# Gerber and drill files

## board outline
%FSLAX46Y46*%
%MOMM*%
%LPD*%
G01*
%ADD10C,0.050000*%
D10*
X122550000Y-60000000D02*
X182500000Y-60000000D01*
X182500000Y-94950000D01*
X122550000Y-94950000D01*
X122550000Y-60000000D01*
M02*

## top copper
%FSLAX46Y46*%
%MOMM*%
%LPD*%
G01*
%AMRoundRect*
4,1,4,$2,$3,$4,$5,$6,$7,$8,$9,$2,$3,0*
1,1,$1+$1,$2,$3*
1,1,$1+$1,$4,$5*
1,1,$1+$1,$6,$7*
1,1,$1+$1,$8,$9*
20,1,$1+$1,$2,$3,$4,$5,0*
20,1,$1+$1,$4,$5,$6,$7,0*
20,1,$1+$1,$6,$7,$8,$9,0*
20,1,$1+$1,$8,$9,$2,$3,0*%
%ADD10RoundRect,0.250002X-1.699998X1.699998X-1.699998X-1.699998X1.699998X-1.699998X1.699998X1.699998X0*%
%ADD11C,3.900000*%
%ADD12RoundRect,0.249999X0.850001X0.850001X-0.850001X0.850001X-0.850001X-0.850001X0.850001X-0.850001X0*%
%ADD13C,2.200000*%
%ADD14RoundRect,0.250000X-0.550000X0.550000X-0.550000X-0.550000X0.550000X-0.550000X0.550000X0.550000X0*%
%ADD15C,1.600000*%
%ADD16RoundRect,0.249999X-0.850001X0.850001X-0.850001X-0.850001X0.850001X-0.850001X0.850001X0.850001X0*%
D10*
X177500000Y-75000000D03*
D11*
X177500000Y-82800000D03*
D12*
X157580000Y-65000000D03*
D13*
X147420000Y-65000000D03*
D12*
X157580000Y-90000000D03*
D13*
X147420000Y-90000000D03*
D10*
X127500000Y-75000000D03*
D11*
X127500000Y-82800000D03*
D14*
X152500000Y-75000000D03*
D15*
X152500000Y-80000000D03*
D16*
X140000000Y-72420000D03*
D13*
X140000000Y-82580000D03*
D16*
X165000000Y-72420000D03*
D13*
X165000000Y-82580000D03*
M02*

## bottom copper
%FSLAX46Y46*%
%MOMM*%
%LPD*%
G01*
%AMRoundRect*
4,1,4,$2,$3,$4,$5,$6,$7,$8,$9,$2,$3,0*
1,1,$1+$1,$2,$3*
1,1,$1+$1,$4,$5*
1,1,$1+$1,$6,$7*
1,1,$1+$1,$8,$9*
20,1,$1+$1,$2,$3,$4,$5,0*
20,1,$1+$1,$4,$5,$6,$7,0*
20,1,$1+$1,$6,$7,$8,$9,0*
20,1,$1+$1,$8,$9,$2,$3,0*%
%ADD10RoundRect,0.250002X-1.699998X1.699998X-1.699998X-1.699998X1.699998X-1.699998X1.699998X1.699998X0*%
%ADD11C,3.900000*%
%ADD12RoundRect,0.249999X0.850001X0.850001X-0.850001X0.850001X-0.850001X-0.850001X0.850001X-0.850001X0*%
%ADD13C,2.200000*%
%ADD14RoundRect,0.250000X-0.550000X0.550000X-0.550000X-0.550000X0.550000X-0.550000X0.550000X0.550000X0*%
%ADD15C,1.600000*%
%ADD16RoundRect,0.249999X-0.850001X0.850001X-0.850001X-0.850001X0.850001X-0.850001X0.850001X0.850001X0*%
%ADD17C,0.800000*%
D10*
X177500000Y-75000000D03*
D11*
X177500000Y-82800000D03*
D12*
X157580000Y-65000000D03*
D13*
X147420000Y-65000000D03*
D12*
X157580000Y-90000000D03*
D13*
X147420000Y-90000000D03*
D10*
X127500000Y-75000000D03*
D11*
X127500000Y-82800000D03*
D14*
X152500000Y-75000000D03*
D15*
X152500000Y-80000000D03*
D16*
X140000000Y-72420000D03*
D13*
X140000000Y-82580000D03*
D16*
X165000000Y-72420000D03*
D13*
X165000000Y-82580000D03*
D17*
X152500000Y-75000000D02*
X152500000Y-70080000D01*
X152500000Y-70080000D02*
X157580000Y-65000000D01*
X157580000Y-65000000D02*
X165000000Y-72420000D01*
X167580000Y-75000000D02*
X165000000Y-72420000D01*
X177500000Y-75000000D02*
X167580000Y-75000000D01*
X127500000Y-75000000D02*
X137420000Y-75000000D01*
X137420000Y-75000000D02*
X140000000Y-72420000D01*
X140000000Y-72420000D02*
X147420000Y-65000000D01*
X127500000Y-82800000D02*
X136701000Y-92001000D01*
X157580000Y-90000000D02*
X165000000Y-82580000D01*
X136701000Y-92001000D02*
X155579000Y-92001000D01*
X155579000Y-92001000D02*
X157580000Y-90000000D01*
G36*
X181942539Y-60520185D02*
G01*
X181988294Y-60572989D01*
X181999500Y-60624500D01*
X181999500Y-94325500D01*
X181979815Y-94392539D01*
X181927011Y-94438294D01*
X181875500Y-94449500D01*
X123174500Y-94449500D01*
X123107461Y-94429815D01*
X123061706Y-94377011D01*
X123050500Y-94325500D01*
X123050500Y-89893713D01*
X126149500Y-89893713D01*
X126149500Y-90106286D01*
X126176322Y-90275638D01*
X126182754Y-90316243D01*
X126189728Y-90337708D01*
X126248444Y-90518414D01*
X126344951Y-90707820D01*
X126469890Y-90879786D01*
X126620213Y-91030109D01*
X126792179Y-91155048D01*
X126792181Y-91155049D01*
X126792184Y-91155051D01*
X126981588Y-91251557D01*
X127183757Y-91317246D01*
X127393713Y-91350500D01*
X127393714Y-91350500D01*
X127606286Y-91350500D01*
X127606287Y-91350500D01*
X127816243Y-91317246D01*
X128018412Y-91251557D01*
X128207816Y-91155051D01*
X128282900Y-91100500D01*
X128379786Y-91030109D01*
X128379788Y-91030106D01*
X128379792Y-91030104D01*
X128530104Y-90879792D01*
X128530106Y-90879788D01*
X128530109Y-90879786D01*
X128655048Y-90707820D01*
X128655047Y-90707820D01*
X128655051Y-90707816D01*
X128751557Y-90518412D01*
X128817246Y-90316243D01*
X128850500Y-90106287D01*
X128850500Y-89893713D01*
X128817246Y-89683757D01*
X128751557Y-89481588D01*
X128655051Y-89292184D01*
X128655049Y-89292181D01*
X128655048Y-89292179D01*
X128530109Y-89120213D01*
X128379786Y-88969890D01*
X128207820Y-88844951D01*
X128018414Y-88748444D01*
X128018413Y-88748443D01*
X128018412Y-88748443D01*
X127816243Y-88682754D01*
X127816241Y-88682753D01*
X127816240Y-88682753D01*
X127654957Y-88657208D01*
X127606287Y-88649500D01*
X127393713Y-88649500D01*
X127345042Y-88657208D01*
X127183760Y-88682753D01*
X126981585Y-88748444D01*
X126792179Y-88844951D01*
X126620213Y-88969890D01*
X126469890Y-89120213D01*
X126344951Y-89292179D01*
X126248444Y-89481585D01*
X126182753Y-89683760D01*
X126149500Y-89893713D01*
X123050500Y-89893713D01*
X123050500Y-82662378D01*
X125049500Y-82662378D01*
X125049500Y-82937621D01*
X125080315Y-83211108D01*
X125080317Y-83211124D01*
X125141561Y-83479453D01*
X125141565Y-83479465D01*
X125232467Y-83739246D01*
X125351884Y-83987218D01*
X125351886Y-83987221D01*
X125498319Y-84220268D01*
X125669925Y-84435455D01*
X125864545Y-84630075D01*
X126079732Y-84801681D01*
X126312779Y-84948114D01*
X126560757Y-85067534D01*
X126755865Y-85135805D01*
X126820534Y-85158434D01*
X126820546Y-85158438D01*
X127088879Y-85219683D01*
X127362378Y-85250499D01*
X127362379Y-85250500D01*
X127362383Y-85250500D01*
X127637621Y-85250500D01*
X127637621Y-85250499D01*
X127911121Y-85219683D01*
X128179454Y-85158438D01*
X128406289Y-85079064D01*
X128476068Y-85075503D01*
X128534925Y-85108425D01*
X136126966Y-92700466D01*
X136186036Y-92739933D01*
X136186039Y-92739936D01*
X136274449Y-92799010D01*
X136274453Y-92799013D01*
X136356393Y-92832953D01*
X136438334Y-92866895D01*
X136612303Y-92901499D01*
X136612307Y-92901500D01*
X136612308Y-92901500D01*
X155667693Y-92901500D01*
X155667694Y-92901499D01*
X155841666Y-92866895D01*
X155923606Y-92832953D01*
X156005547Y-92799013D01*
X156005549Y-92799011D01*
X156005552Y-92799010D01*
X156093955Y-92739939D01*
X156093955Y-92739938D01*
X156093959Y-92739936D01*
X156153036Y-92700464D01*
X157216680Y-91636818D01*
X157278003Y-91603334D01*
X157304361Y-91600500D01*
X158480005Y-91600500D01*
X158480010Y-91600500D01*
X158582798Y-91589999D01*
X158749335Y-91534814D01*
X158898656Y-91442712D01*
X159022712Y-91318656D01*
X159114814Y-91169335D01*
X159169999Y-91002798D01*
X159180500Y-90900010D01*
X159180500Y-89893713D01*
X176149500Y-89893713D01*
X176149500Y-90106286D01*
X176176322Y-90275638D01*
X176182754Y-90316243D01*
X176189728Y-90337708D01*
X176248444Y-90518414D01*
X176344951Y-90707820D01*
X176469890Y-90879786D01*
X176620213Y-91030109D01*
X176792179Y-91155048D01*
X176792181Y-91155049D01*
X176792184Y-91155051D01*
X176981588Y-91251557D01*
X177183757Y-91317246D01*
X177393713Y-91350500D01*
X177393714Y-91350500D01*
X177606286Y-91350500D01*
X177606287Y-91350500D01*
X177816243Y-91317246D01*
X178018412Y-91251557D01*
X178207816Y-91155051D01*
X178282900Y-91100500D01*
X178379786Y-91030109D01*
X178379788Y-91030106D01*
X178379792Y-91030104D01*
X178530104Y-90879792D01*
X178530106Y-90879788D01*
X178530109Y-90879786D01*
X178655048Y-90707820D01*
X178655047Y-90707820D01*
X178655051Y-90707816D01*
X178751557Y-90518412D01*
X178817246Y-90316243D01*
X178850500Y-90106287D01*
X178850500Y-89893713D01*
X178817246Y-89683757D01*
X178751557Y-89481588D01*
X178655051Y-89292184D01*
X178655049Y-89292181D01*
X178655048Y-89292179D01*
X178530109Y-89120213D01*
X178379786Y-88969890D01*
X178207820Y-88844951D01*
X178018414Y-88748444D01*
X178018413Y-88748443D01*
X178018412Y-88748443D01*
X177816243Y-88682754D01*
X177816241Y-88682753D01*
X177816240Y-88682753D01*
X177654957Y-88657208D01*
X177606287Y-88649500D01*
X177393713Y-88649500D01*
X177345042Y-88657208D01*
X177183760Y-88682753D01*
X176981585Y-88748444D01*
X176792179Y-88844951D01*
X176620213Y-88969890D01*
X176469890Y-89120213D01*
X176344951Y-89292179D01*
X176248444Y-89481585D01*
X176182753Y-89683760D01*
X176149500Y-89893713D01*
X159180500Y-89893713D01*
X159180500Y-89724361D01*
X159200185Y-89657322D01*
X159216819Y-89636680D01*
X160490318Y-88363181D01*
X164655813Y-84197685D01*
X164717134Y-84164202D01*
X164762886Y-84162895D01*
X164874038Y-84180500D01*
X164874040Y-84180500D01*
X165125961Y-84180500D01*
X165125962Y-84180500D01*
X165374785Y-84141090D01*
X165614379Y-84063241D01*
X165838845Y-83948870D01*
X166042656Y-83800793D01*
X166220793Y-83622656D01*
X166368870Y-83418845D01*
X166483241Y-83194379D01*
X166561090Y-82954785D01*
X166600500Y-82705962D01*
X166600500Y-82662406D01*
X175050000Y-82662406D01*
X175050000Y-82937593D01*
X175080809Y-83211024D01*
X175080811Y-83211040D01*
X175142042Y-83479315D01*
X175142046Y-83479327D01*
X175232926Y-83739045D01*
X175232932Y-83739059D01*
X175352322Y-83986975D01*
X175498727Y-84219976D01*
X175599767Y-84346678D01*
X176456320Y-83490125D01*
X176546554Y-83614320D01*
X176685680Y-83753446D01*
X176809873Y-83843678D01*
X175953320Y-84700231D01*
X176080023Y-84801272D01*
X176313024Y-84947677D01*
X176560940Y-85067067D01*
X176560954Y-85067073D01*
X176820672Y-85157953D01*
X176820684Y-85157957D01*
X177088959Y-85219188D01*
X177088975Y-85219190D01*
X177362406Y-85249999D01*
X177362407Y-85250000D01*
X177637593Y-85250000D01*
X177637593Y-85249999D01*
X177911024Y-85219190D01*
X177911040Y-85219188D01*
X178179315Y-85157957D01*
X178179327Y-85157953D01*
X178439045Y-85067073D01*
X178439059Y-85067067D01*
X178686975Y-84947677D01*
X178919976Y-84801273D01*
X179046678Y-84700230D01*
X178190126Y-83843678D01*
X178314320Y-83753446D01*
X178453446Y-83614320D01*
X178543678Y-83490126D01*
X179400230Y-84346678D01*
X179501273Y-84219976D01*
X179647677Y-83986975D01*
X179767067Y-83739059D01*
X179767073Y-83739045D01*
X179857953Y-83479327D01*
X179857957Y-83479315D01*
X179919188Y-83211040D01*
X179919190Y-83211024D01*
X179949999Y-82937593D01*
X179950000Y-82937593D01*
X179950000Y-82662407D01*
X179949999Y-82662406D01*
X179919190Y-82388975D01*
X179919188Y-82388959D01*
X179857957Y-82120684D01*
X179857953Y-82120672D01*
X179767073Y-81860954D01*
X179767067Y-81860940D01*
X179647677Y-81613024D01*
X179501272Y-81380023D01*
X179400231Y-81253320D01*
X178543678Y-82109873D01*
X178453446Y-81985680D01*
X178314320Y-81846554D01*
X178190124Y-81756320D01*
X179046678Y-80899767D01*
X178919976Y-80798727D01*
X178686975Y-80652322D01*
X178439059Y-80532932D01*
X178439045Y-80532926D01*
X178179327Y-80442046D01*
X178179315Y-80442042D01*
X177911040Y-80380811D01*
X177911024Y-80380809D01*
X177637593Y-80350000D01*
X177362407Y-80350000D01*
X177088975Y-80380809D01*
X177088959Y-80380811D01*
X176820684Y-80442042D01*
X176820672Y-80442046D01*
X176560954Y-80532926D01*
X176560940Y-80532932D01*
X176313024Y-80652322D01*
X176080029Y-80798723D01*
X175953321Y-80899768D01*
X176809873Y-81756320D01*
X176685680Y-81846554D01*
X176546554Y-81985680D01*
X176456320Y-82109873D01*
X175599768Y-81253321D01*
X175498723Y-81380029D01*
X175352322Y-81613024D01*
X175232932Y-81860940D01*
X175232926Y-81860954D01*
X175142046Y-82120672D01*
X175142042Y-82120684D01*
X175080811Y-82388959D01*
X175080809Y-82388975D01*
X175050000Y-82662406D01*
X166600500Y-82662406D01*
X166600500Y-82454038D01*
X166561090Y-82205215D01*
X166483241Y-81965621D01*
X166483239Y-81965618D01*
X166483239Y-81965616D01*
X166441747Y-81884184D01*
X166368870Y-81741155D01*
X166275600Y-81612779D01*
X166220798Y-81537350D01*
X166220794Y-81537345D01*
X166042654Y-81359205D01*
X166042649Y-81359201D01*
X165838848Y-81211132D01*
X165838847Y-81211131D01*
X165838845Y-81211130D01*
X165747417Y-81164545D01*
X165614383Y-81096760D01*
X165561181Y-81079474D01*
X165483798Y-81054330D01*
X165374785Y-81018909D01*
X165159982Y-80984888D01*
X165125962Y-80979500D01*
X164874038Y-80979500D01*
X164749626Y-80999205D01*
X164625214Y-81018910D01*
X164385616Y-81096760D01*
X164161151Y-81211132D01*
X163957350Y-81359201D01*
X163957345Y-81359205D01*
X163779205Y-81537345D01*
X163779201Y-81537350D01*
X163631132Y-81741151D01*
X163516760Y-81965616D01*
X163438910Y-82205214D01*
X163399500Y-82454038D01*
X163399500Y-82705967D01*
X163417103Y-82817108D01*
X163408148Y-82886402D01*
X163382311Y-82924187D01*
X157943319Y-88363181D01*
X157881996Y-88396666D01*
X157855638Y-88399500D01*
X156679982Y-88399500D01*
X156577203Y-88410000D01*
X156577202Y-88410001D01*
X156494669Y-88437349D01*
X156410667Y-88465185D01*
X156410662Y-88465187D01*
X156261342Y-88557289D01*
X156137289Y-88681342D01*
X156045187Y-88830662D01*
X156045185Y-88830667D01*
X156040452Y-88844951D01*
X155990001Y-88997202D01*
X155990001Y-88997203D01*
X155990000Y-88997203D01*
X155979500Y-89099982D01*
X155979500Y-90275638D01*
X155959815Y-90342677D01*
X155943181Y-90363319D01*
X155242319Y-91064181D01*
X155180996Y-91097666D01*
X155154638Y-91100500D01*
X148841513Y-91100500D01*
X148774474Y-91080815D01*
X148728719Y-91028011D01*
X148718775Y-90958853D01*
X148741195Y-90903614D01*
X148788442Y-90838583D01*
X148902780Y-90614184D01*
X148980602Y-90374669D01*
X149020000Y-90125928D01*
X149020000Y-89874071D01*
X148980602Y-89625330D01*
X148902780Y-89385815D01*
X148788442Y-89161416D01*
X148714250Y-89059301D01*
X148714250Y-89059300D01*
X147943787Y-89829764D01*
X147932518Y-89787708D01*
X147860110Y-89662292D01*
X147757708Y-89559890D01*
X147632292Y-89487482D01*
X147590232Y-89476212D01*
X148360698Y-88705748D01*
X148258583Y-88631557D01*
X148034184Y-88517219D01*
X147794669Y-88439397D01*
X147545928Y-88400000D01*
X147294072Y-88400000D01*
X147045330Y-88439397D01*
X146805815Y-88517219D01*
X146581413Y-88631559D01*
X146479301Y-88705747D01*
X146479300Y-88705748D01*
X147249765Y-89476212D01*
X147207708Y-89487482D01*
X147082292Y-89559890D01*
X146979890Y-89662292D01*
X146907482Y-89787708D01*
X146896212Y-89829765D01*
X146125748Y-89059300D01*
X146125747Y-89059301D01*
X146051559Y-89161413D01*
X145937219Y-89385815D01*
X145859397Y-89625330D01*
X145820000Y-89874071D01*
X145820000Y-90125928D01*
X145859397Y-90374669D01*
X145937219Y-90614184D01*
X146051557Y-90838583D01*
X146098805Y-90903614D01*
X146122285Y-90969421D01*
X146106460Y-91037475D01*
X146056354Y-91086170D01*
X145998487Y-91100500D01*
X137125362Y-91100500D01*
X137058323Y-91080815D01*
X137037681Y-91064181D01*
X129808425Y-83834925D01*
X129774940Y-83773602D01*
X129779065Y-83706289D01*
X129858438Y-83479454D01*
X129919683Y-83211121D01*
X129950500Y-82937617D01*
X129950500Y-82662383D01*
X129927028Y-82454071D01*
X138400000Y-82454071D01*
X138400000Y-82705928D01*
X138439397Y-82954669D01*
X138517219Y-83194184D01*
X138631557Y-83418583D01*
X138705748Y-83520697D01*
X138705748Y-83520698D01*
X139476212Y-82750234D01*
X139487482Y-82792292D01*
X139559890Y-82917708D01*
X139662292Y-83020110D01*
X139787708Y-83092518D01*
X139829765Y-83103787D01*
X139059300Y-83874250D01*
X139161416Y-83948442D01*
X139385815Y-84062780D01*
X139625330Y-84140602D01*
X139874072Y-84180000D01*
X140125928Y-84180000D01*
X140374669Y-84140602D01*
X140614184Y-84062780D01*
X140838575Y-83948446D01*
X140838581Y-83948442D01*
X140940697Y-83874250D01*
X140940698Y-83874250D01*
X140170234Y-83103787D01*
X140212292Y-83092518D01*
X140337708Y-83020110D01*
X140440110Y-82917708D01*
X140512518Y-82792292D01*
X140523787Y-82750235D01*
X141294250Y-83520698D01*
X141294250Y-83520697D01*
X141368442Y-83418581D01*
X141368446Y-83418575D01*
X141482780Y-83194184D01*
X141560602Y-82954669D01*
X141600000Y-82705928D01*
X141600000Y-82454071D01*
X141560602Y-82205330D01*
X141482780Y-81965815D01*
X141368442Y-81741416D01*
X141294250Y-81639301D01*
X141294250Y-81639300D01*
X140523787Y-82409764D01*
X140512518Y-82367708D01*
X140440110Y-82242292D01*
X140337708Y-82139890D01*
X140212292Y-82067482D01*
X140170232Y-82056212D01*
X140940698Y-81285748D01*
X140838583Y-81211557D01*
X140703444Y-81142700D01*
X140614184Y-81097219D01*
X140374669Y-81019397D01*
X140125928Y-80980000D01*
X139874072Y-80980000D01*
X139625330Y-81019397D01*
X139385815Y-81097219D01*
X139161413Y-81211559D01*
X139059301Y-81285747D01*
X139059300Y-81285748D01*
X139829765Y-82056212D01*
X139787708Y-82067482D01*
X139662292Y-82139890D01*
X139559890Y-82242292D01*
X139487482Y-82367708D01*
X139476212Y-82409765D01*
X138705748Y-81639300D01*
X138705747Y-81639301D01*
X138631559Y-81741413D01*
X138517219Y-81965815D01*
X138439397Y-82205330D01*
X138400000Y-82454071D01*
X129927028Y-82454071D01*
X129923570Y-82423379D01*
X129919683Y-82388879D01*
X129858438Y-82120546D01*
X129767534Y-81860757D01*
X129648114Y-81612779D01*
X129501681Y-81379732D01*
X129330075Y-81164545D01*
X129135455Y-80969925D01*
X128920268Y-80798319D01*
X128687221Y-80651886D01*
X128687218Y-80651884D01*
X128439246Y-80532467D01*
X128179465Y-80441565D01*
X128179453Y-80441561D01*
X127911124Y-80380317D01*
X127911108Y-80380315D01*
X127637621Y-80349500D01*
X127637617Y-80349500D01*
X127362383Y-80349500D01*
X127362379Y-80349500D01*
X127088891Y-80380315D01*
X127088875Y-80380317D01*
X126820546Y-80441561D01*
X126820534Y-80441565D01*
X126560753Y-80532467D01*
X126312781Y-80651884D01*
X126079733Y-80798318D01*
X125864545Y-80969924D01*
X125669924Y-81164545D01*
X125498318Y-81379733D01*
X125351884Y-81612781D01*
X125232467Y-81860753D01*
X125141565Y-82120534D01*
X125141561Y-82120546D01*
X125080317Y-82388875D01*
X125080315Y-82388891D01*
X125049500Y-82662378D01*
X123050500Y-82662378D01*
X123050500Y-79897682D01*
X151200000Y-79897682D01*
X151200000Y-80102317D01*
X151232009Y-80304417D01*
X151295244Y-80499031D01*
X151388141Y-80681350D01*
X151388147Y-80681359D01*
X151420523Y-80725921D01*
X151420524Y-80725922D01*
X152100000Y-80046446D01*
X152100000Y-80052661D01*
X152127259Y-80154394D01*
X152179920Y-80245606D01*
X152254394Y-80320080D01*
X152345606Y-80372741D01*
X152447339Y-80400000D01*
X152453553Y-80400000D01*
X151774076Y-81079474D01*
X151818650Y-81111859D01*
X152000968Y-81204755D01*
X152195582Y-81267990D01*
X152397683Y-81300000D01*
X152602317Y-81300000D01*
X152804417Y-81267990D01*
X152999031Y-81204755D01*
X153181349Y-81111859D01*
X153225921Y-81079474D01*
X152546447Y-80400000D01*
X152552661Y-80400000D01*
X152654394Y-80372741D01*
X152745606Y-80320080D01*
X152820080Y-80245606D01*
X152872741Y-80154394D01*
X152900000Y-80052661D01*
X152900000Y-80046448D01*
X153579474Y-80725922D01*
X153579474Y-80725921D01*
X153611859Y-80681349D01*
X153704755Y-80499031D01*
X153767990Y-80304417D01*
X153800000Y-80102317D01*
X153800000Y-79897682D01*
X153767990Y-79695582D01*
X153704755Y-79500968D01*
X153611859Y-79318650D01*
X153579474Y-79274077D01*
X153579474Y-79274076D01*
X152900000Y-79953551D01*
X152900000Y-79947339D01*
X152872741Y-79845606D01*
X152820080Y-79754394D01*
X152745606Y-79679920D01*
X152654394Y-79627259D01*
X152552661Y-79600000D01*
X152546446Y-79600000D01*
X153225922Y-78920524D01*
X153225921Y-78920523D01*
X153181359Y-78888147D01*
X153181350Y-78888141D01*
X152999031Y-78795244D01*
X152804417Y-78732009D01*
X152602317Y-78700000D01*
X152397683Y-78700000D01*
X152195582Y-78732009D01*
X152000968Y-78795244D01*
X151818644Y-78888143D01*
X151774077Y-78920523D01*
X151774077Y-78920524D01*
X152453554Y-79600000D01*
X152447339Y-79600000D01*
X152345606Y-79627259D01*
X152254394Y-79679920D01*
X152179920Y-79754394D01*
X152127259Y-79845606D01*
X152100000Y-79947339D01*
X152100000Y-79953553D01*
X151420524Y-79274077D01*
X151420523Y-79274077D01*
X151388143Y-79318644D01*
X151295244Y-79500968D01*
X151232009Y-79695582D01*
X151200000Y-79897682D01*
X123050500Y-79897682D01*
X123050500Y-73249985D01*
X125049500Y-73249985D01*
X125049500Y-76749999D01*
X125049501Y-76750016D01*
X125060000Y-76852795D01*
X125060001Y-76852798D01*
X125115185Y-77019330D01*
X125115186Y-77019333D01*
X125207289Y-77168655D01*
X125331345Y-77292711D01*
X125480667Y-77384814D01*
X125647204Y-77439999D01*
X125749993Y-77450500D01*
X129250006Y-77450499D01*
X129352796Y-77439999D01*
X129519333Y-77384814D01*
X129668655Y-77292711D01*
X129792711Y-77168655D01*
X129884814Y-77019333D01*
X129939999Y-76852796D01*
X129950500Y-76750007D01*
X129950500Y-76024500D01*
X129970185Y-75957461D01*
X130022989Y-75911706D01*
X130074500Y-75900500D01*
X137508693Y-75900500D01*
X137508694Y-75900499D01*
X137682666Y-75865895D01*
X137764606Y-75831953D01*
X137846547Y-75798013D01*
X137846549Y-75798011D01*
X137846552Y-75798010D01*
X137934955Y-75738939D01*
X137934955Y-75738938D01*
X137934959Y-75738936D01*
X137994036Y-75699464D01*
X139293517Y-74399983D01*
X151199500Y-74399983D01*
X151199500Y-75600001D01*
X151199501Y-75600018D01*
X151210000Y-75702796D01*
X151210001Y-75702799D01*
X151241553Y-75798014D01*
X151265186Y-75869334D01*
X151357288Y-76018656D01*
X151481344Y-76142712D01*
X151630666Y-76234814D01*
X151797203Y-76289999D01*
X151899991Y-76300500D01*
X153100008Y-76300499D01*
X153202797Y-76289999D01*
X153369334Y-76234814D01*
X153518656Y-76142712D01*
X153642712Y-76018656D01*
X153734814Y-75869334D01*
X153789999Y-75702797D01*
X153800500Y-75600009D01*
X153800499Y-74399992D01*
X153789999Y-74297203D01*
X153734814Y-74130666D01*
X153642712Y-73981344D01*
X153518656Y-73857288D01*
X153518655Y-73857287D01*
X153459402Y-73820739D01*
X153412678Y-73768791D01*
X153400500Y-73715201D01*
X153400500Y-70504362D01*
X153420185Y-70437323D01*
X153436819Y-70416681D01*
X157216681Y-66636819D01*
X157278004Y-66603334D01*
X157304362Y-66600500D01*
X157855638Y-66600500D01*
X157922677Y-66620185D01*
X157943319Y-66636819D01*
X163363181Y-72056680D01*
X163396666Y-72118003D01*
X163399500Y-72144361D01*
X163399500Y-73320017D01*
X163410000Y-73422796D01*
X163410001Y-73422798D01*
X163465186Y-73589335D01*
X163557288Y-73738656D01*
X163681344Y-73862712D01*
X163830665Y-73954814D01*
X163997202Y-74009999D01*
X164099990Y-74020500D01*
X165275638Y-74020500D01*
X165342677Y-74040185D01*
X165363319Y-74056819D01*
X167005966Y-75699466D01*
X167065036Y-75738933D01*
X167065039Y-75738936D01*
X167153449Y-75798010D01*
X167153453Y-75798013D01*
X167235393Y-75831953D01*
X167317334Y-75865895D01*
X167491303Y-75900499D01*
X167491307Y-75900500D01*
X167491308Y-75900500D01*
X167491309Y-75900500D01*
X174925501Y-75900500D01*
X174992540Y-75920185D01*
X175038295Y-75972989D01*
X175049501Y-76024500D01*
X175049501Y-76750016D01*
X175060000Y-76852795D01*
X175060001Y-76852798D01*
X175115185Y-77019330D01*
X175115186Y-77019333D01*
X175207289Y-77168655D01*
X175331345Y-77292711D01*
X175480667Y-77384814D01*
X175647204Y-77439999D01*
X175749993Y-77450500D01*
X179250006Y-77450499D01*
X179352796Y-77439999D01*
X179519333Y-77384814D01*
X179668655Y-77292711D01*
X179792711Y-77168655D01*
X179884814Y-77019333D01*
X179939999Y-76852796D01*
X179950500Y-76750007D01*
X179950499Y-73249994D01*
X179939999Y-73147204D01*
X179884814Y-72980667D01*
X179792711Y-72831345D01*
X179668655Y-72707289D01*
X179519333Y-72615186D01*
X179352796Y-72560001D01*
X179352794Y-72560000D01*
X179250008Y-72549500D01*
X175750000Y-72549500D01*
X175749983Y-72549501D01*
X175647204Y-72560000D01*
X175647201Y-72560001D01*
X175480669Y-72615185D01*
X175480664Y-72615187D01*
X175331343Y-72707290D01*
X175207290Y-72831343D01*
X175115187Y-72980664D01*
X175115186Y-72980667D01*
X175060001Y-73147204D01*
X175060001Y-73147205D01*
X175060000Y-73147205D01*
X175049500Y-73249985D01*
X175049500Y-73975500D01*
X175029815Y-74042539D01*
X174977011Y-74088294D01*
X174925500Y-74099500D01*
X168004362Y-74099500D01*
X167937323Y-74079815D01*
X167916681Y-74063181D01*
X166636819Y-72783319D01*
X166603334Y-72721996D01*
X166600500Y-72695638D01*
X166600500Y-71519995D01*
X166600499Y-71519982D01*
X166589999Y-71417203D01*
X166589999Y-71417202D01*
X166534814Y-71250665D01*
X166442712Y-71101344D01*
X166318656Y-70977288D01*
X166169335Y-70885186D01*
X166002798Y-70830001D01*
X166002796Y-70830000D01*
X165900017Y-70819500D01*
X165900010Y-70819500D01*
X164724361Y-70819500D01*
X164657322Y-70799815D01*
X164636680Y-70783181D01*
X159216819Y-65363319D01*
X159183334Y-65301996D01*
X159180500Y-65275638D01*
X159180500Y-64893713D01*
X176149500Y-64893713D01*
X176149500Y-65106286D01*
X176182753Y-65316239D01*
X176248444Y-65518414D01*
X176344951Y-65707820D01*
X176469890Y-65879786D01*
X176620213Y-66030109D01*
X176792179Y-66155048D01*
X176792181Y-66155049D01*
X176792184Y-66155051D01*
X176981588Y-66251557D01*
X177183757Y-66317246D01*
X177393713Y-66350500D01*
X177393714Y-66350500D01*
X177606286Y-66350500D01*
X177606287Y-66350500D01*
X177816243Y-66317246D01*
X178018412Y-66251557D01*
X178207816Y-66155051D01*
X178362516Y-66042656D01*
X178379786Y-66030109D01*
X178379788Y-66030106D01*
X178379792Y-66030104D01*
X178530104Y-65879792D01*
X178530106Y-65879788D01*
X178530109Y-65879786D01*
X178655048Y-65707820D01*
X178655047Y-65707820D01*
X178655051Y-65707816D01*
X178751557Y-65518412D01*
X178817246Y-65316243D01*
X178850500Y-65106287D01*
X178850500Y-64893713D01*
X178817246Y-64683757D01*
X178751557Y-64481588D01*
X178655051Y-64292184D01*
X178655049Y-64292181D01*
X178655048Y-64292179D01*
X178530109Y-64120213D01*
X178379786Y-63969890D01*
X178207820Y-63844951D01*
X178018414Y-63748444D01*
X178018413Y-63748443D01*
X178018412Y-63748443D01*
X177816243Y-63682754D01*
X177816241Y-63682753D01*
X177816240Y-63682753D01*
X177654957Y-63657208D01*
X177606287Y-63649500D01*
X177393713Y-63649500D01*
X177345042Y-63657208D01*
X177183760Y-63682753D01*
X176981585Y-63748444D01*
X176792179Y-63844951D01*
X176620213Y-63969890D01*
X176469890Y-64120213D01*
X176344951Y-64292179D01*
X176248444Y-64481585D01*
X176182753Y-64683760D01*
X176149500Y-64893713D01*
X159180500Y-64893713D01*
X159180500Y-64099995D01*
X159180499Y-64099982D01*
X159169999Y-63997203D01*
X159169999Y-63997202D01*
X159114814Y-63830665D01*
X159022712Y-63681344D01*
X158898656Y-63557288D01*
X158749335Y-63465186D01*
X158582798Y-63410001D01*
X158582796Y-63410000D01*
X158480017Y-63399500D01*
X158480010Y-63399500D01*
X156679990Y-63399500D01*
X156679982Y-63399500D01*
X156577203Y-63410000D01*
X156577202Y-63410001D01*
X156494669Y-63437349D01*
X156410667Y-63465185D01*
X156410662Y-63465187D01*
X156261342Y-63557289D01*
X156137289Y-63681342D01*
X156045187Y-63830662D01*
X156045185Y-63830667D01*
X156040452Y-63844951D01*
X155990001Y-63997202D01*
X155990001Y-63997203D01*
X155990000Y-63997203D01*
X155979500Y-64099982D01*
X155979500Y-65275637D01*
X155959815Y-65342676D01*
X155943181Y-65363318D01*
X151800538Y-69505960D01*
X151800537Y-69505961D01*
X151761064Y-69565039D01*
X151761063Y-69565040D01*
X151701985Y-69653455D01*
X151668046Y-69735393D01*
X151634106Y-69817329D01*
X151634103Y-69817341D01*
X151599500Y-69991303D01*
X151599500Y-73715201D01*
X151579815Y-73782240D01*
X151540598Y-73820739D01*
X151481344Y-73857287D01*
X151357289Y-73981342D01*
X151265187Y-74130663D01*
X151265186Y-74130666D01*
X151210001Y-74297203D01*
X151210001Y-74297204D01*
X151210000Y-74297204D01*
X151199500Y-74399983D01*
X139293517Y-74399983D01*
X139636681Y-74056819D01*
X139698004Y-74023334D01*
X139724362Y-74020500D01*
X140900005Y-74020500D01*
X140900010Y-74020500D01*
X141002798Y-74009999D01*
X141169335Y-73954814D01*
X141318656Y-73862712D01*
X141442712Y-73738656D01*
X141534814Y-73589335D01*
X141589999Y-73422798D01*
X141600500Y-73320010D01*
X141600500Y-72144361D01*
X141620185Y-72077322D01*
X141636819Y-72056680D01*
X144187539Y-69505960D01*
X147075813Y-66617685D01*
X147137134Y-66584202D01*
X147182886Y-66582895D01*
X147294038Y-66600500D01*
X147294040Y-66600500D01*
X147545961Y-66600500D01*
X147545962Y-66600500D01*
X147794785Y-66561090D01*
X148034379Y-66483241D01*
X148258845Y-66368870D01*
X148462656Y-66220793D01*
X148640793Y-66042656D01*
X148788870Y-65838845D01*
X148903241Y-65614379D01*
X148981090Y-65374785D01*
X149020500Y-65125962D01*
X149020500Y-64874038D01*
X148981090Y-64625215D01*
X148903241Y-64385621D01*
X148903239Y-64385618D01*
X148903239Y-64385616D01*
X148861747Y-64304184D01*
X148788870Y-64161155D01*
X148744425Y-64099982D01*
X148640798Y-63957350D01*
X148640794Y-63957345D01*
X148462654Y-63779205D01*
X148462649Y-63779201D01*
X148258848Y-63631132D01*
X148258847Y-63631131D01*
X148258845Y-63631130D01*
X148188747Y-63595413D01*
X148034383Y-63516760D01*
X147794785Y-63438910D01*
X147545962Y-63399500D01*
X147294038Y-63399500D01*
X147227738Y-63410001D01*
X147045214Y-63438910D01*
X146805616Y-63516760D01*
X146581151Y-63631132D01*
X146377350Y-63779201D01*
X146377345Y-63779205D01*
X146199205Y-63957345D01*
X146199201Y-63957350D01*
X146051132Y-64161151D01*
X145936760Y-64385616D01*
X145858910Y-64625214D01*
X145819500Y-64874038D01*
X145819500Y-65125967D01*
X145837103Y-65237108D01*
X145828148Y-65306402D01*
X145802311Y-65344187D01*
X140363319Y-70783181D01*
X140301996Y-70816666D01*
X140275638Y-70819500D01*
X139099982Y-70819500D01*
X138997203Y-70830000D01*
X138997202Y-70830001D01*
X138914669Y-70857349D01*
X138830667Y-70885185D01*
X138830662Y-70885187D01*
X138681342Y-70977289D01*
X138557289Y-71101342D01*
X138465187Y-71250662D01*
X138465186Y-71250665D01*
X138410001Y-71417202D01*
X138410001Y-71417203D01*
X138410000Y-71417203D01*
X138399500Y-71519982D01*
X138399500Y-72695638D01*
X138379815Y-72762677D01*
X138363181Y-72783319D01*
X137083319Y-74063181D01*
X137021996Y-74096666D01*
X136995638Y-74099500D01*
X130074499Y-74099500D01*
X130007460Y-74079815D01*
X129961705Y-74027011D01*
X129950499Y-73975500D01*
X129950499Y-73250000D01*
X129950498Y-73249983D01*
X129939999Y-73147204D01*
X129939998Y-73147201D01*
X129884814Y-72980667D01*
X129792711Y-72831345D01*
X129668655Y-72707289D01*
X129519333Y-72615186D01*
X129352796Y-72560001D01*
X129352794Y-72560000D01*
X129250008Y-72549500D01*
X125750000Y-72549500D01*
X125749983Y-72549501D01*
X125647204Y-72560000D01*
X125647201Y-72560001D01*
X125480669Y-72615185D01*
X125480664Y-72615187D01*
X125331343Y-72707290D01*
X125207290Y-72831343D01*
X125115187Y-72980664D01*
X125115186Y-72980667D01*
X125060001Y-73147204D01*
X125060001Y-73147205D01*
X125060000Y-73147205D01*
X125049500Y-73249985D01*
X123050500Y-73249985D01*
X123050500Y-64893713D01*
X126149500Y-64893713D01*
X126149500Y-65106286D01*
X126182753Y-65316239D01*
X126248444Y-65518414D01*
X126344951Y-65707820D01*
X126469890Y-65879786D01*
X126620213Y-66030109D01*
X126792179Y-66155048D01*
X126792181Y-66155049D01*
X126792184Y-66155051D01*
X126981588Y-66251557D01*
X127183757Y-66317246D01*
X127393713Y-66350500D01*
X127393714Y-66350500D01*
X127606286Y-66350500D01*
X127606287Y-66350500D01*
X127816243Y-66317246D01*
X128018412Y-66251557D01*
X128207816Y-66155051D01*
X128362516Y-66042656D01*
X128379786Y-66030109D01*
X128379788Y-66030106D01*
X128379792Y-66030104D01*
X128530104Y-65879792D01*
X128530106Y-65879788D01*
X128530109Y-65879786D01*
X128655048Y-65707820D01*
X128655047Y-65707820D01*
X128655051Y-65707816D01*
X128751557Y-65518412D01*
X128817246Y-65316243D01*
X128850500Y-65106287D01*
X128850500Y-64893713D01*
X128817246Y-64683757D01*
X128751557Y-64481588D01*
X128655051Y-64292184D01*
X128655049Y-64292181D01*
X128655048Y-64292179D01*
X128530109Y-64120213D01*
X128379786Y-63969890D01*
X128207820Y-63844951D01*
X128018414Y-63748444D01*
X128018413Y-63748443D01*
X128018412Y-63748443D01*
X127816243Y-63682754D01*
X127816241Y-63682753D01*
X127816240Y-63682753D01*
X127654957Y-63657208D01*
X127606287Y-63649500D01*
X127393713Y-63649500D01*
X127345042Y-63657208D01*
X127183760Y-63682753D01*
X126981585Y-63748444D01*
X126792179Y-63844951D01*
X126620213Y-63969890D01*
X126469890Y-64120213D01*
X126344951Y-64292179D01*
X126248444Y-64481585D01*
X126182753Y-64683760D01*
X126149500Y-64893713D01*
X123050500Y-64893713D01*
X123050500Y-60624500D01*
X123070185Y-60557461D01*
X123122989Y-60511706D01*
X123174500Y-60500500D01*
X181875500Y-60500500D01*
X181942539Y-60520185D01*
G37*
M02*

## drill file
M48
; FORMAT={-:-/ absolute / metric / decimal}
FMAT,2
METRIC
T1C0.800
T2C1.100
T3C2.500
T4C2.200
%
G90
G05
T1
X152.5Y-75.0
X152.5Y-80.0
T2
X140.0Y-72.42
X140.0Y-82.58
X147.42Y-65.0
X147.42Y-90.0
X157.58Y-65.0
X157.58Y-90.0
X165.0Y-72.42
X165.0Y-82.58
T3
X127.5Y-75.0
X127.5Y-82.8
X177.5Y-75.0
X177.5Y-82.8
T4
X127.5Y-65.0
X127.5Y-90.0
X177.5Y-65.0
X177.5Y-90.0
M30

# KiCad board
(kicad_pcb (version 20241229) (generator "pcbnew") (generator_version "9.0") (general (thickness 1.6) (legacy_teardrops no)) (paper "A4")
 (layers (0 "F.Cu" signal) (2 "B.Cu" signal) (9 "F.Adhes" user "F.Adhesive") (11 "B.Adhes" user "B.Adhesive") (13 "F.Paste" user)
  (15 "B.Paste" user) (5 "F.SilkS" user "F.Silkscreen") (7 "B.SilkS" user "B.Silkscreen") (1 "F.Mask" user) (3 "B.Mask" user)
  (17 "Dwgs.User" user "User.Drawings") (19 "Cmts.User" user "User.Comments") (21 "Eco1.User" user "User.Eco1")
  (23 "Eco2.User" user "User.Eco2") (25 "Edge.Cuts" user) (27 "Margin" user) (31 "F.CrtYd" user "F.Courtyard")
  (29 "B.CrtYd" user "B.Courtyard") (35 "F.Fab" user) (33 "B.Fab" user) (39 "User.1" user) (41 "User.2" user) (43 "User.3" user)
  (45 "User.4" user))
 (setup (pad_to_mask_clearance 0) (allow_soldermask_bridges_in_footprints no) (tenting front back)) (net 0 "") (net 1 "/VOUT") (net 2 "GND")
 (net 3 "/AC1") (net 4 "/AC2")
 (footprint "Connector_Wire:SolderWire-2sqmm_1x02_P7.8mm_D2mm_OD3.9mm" (layer "F.Cu") (at 177.5 75 -90)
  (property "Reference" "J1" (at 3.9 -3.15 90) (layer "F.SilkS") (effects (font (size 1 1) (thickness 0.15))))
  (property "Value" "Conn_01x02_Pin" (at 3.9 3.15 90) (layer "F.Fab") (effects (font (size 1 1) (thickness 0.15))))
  (pad "1" thru_hole roundrect (at 0 0 270) (size 3.9 3.9) (drill 2.5) (layers "*.Cu" "*.Mask") (remove_unused_layers no)
   (roundrect_rratio 0.064103) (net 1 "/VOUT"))
  (pad "2" thru_hole circle (at 7.8 0 270) (size 3.9 3.9) (drill 2.5) (layers "*.Cu" "*.Mask") (remove_unused_layers no) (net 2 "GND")))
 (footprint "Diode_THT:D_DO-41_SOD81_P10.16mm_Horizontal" (layer "F.Cu") (at 157.58 65 180)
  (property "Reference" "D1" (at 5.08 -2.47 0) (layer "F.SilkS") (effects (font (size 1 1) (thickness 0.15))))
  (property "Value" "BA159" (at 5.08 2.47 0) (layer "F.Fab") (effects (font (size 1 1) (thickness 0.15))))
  (pad "1" thru_hole roundrect (at 0 0 180) (size 2.2 2.2) (drill 1.1) (layers "*.Cu" "*.Mask") (remove_unused_layers no)
   (roundrect_rratio 0.113636) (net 1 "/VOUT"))
  (pad "2" thru_hole circle (at 10.16 0 180) (size 2.2 2.2) (drill 1.1) (layers "*.Cu" "*.Mask") (remove_unused_layers no) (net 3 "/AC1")))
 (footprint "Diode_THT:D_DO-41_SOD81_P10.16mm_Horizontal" (layer "F.Cu") (at 157.58 90 180)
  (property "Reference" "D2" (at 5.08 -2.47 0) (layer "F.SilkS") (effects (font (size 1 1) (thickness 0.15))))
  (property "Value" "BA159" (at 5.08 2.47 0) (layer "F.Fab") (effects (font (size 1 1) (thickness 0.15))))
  (pad "1" thru_hole roundrect (at 0 0 180) (size 2.2 2.2) (drill 1.1) (layers "*.Cu" "*.Mask") (remove_unused_layers no)
   (roundrect_rratio 0.113636) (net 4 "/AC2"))
  (pad "2" thru_hole circle (at 10.16 0 180) (size 2.2 2.2) (drill 1.1) (layers "*.Cu" "*.Mask") (remove_unused_layers no) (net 2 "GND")))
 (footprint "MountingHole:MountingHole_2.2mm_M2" (layer "F.Cu") (at 127.5 65)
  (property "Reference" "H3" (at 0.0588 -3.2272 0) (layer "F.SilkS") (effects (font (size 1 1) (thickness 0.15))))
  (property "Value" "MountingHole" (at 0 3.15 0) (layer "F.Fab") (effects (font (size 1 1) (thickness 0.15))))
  (pad "" np_thru_hole circle (at 0 0) (size 2.2 2.2) (drill 2.2) (layers "*.Cu" "*.Mask")))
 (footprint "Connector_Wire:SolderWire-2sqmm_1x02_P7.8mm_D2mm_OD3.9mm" (layer "F.Cu") (at 127.5 75 -90)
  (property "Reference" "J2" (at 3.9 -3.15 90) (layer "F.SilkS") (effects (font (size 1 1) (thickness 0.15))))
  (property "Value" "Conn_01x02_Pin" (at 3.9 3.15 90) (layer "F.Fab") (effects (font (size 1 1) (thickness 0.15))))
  (pad "1" thru_hole roundrect (at 0 0 270) (size 3.9 3.9) (drill 2.5) (layers "*.Cu" "*.Mask") (remove_unused_layers no)
   (roundrect_rratio 0.064103) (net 3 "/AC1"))
  (pad "2" thru_hole circle (at 7.8 0 270) (size 3.9 3.9) (drill 2.5) (layers "*.Cu" "*.Mask") (remove_unused_layers no) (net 4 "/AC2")))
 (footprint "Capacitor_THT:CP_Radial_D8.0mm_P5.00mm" (layer "F.Cu") (at 152.5 75 -90)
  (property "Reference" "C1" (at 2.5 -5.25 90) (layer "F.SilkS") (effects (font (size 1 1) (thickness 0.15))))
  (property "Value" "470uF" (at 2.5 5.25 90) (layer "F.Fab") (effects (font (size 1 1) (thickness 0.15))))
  (pad "1" thru_hole roundrect (at 0 0 270) (size 1.6 1.6) (drill 0.8) (layers "*.Cu" "*.Mask") (remove_unused_layers no)
   (roundrect_rratio 0.15625) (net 1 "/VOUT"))
  (pad "2" thru_hole circle (at 5 0 270) (size 1.6 1.6) (drill 0.8) (layers "*.Cu" "*.Mask") (remove_unused_layers no) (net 2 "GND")))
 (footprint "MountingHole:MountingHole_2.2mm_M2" (layer "F.Cu") (at 177.5 90)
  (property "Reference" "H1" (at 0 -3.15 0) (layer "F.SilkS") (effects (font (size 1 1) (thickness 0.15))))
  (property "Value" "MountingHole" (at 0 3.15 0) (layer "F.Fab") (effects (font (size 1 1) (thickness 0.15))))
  (pad "" np_thru_hole circle (at 0 0) (size 2.2 2.2) (drill 2.2) (layers "*.Cu" "*.Mask")))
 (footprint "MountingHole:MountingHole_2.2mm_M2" (layer "F.Cu") (at 127.5 90)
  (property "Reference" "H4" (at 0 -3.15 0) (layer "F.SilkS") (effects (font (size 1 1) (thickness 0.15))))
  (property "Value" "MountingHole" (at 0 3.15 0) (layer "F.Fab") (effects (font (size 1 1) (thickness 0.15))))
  (pad "" np_thru_hole circle (at 0 0) (size 2.2 2.2) (drill 2.2) (layers "*.Cu" "*.Mask")))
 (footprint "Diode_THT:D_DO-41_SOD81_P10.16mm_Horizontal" (layer "F.Cu") (at 140 72.42 -90)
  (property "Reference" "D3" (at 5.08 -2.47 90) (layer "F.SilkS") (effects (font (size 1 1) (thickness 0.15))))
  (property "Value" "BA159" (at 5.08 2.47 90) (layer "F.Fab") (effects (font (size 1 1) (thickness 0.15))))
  (pad "1" thru_hole roundrect (at 0 0 270) (size 2.2 2.2) (drill 1.1) (layers "*.Cu" "*.Mask") (remove_unused_layers no)
   (roundrect_rratio 0.113636) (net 3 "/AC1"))
  (pad "2" thru_hole circle (at 10.16 0 270) (size 2.2 2.2) (drill 1.1) (layers "*.Cu" "*.Mask") (remove_unused_layers no) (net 2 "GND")))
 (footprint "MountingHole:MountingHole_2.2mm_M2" (layer "F.Cu") (at 177.5 65)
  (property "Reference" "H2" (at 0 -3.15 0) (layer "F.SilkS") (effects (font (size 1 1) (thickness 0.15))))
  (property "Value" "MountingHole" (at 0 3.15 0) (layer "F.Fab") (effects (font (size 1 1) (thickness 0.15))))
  (pad "" np_thru_hole circle (at 0 0) (size 2.2 2.2) (drill 2.2) (layers "*.Cu" "*.Mask")))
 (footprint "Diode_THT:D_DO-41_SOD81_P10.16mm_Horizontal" (layer "F.Cu") (at 165 72.42 -90)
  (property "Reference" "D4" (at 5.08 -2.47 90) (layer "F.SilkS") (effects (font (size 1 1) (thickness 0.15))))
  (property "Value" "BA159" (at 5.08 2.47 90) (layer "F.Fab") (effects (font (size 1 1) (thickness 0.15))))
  (pad "1" thru_hole roundrect (at 0 0 270) (size 2.2 2.2) (drill 1.1) (layers "*.Cu" "*.Mask") (remove_unused_layers no)
   (roundrect_rratio 0.113636) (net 1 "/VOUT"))
  (pad "2" thru_hole circle (at 10.16 0 270) (size 2.2 2.2) (drill 1.1) (layers "*.Cu" "*.Mask") (remove_unused_layers no) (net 4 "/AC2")))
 (gr_rect (start 122.55 60) (end 182.5 94.95) (stroke (width 0.05) (type default)) (fill no) (layer "Edge.Cuts"))
 (segment (start 152.5 75) (end 152.5 70.08) (width 0.8) (layer "B.Cu") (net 1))
 (segment (start 152.5 70.08) (end 157.58 65) (width 0.8) (layer "B.Cu") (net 1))
 (segment (start 157.58 65) (end 165 72.42) (width 0.8) (layer "B.Cu") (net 1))
 (segment (start 167.58 75) (end 165 72.42) (width 0.8) (layer "B.Cu") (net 1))
 (segment (start 177.5 75) (end 167.58 75) (width 0.8) (layer "B.Cu") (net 1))
 (segment (start 127.5 75) (end 137.42 75) (width 0.8) (layer "B.Cu") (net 3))
 (segment (start 137.42 75) (end 140 72.42) (width 0.8) (layer "B.Cu") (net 3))
 (segment (start 140 72.42) (end 147.42 65) (width 0.8) (layer "B.Cu") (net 3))
 (segment (start 127.5 82.8) (end 136.701 92.001) (width 0.8) (layer "B.Cu") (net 4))
 (segment (start 157.58 90) (end 165 82.58) (width 0.8) (layer "B.Cu") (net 4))
 (segment (start 136.701 92.001) (end 155.579 92.001) (width 0.8) (layer "B.Cu") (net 4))
 (segment (start 155.579 92.001) (end 157.58 90) (width 0.8) (layer "B.Cu") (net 4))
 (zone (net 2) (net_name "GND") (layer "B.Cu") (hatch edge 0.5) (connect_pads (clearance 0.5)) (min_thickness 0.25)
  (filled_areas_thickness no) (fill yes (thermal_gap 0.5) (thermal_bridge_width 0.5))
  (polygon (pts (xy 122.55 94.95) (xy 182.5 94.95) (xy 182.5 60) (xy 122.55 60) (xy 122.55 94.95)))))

